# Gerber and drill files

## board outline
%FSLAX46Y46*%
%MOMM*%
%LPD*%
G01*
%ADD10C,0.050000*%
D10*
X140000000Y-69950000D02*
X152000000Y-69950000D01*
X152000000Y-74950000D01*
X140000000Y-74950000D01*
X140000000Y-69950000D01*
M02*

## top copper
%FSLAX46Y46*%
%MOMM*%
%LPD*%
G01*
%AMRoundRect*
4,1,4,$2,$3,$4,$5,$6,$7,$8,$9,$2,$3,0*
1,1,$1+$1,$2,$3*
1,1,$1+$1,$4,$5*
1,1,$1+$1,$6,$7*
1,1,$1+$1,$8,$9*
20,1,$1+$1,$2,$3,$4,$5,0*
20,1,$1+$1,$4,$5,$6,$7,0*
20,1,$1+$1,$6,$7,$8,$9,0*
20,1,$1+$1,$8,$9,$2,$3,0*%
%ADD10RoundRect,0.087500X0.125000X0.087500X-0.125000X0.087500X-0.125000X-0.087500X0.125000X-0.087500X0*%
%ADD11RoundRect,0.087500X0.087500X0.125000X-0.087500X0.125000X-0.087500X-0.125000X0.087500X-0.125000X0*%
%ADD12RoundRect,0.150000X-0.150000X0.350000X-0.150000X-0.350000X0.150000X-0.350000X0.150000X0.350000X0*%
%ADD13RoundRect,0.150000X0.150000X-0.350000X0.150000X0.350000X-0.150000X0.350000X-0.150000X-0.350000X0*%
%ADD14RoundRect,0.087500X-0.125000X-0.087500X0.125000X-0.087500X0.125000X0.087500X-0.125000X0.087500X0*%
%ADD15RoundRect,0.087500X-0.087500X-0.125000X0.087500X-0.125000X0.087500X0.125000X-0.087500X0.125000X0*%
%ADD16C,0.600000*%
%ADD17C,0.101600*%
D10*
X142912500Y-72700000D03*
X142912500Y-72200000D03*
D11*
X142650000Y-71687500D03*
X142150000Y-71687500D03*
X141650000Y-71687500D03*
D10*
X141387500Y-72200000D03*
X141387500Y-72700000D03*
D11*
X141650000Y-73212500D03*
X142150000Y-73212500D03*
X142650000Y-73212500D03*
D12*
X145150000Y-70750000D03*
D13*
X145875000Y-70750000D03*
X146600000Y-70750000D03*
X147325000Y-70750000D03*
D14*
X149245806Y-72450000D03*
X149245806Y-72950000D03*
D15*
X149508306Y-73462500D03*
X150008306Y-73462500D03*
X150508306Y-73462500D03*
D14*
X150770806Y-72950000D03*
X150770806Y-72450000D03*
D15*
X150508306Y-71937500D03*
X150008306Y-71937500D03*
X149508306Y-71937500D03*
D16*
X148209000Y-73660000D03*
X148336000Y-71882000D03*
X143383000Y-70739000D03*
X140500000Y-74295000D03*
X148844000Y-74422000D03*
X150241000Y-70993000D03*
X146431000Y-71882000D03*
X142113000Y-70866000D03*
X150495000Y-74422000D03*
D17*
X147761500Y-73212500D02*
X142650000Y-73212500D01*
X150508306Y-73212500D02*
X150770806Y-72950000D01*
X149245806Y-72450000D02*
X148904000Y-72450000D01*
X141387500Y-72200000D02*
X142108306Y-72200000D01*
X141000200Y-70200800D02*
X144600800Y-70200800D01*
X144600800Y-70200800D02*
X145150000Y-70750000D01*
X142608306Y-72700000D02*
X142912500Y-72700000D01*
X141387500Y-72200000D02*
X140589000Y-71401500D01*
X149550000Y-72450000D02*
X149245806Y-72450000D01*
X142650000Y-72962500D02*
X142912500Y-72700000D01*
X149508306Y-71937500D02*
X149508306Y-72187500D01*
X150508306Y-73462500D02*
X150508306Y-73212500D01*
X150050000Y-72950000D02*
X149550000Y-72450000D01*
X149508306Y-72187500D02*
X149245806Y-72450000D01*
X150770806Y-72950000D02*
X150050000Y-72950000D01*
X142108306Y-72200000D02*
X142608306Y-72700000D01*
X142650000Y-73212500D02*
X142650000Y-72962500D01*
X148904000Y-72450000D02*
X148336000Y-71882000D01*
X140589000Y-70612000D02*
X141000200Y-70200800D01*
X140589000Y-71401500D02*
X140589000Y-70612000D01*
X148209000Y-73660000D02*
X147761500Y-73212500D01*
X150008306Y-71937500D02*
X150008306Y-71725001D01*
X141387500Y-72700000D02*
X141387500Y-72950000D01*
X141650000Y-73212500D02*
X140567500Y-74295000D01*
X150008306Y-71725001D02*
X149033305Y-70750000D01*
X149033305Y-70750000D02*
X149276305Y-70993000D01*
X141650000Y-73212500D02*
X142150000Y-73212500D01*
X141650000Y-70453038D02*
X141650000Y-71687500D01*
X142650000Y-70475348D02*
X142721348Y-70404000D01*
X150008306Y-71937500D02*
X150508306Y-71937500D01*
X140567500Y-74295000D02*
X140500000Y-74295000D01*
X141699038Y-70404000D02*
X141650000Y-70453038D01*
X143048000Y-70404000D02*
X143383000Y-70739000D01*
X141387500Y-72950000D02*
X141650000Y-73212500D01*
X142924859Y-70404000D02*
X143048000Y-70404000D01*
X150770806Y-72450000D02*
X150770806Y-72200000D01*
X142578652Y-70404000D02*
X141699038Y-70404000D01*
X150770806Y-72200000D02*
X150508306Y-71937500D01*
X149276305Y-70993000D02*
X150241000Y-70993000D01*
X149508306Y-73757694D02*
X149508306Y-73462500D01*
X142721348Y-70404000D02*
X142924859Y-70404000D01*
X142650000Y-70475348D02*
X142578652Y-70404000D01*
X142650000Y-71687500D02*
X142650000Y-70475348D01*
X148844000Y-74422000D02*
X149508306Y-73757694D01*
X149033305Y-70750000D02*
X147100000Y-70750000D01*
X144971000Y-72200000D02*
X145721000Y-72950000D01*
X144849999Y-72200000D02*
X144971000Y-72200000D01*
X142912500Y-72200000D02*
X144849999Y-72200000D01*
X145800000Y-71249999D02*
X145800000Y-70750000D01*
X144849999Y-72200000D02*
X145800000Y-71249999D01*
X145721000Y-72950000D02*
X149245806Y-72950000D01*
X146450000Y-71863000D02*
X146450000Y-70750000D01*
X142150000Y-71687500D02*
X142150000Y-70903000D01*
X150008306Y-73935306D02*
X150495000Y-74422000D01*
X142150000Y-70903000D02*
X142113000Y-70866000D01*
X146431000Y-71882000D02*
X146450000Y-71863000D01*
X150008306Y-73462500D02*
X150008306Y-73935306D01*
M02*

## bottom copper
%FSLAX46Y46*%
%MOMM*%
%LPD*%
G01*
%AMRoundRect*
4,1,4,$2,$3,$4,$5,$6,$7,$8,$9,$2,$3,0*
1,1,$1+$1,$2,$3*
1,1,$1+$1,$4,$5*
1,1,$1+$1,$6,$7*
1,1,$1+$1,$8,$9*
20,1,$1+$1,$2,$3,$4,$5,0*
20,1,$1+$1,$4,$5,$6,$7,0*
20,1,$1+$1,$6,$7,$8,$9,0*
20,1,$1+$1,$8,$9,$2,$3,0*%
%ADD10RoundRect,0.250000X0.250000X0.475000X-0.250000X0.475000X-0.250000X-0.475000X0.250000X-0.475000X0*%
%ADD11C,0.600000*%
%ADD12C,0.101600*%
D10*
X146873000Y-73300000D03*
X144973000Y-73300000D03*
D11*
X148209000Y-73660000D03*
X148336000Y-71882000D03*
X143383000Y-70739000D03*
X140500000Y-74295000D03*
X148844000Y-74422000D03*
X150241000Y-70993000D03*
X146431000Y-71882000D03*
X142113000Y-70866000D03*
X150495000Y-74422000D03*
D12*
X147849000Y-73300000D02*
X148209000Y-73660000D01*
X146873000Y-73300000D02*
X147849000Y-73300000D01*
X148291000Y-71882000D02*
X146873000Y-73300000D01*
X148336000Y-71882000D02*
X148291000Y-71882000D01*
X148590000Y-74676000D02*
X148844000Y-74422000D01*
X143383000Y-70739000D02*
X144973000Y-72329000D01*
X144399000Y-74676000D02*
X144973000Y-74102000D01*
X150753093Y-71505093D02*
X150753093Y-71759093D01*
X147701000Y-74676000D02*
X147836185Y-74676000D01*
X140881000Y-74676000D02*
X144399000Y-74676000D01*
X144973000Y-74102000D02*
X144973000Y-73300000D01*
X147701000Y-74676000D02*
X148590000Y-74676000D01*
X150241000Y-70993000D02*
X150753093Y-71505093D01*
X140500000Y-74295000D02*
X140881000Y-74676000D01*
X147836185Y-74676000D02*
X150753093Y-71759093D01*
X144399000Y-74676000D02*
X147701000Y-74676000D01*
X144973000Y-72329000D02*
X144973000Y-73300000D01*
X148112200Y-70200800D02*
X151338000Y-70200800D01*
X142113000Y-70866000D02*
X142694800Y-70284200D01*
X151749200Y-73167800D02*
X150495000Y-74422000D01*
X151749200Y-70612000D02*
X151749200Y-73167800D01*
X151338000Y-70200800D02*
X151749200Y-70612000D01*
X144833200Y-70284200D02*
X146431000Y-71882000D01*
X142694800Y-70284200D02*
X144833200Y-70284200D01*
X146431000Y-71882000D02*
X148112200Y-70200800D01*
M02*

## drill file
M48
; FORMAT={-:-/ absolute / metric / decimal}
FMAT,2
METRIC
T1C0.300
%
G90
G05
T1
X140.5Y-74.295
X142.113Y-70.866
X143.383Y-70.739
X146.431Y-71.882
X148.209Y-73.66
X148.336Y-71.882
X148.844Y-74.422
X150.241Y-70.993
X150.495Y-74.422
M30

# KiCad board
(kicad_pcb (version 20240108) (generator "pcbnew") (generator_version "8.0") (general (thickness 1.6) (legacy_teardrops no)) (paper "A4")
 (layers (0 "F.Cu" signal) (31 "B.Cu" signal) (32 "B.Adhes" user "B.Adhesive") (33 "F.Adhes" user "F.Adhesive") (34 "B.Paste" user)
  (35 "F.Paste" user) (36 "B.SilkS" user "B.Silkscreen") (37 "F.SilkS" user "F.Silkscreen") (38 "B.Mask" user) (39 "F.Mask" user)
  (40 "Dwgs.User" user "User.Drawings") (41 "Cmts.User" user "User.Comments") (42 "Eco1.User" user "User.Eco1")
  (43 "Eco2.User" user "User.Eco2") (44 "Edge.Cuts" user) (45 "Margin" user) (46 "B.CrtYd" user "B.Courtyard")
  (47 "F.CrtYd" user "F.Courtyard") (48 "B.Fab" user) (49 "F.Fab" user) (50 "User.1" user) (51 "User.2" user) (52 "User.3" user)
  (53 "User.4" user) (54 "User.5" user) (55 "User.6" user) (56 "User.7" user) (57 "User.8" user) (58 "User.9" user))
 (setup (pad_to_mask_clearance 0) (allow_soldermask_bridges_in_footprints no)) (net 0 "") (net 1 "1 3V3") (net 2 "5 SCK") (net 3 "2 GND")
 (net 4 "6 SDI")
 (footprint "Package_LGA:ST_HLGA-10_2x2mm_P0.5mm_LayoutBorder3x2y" (layer "F.Cu") (at 142.15 72.45 180)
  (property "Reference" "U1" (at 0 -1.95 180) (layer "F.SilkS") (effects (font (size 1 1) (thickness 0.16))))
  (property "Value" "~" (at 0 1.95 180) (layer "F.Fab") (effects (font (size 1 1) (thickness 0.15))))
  (pad "1" smd roundrect (at -0.7625 -0.25 180) (size 0.425 0.35) (layers "F.Cu" "F.Paste" "F.Mask") (roundrect_rratio 0.25) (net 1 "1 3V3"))
  (pad "2" smd roundrect (at -0.7625 0.25 180) (size 0.425 0.35) (layers "F.Cu" "F.Paste" "F.Mask") (roundrect_rratio 0.25) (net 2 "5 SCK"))
  (pad "3" smd roundrect (at -0.5 0.7625 180) (size 0.35 0.425) (layers "F.Cu" "F.Paste" "F.Mask") (roundrect_rratio 0.25) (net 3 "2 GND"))
  (pad "4" smd roundrect (at 0 0.7625 180) (size 0.35 0.425) (layers "F.Cu" "F.Paste" "F.Mask") (roundrect_rratio 0.25) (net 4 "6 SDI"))
  (pad "5" smd roundrect (at 0.5 0.7625 180) (size 0.35 0.425) (layers "F.Cu" "F.Paste" "F.Mask") (roundrect_rratio 0.25) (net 3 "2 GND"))
  (pad "6" smd roundrect (at 0.7625 0.25 180) (size 0.425 0.35) (layers "F.Cu" "F.Paste" "F.Mask") (roundrect_rratio 0.25) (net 1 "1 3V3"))
  (pad "7" smd roundrect (at 0.7625 -0.25 180) (size 0.425 0.35) (layers "F.Cu" "F.Paste" "F.Mask") (roundrect_rratio 0.25) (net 3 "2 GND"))
  (pad "8" smd roundrect (at 0.5 -0.7625 180) (size 0.35 0.425) (layers "F.Cu" "F.Paste" "F.Mask") (roundrect_rratio 0.25) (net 3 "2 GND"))
  (pad "9" smd roundrect (at 0 -0.7625 180) (size 0.35 0.425) (layers "F.Cu" "F.Paste" "F.Mask") (roundrect_rratio 0.25) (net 3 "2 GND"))
  (pad "10" smd roundrect (at -0.5 -0.7625 180) (size 0.35 0.425) (layers "F.Cu" "F.Paste" "F.Mask") (roundrect_rratio 0.25) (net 1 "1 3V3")))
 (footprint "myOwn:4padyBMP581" (layer "F.Cu") (at 144.95 65)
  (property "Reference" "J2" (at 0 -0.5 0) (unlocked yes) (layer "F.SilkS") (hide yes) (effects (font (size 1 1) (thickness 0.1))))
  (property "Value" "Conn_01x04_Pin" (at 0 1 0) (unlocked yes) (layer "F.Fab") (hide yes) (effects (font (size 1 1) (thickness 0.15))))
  (pad "1" smd roundrect (at 0.2 5.75 270) (size 1 0.6) (layers "F.Cu" "F.Paste" "F.Mask") (roundrect_rratio 0.25) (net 1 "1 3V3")
   (thermal_bridge_angle 45))
  (pad "2" smd roundrect (at 0.925 5.75 90) (size 1 0.6) (layers "F.Cu" "F.Paste" "F.Mask") (roundrect_rratio 0.25) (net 2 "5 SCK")
   (thermal_bridge_angle 45))
  (pad "3" smd roundrect (at 1.65 5.75 90) (size 1 0.6) (layers "F.Cu" "F.Paste" "F.Mask") (roundrect_rratio 0.25) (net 4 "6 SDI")
   (thermal_bridge_angle 45))
  (pad "4" smd roundrect (at 2.375 5.75 90) (size 1 0.6) (layers "F.Cu" "F.Paste" "F.Mask") (roundrect_rratio 0.25) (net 3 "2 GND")
   (thermal_bridge_angle 45)))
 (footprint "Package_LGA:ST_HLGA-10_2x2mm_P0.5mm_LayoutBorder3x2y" (layer "F.Cu") (at 150.008306 72.7)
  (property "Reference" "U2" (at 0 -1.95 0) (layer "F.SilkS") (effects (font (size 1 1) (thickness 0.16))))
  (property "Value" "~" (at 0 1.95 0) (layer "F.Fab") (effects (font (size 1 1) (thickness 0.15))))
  (pad "1" smd roundrect (at -0.7625 -0.25) (size 0.425 0.35) (layers "F.Cu" "F.Paste" "F.Mask") (roundrect_rratio 0.25) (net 1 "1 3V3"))
  (pad "2" smd roundrect (at -0.7625 0.25) (size 0.425 0.35) (layers "F.Cu" "F.Paste" "F.Mask") (roundrect_rratio 0.25) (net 2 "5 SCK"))
  (pad "3" smd roundrect (at -0.5 0.7625) (size 0.35 0.425) (layers "F.Cu" "F.Paste" "F.Mask") (roundrect_rratio 0.25) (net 3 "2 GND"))
  (pad "4" smd roundrect (at 0 0.7625) (size 0.35 0.425) (layers "F.Cu" "F.Paste" "F.Mask") (roundrect_rratio 0.25) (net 4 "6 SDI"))
  (pad "5" smd roundrect (at 0.5 0.7625) (size 0.35 0.425) (layers "F.Cu" "F.Paste" "F.Mask") (roundrect_rratio 0.25) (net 1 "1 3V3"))
  (pad "6" smd roundrect (at 0.7625 0.25) (size 0.425 0.35) (layers "F.Cu" "F.Paste" "F.Mask") (roundrect_rratio 0.25) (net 1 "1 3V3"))
  (pad "7" smd roundrect (at 0.7625 -0.25) (size 0.425 0.35) (layers "F.Cu" "F.Paste" "F.Mask") (roundrect_rratio 0.25) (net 3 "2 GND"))
  (pad "8" smd roundrect (at 0.5 -0.7625) (size 0.35 0.425) (layers "F.Cu" "F.Paste" "F.Mask") (roundrect_rratio 0.25) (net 3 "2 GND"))
  (pad "9" smd roundrect (at 0 -0.7625) (size 0.35 0.425) (layers "F.Cu" "F.Paste" "F.Mask") (roundrect_rratio 0.25) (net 3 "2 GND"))
  (pad "10" smd roundrect (at -0.5 -0.7625) (size 0.35 0.425) (layers "F.Cu" "F.Paste" "F.Mask") (roundrect_rratio 0.25) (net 1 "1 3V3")))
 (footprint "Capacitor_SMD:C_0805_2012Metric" (layer "B.Cu") (at 145.923 73.3 180)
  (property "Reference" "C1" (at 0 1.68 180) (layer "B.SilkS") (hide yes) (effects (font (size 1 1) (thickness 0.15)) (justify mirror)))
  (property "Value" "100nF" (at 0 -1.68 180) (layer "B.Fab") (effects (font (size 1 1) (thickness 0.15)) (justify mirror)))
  (pad "1" smd roundrect (at -0.95 0 180) (size 1 1.45) (layers "B.Cu" "B.Paste" "B.Mask") (roundrect_rratio 0.25) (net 1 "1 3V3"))
  (pad "2" smd roundrect (at 0.95 0 180) (size 1 1.45) (layers "B.Cu" "B.Paste" "B.Mask") (roundrect_rratio 0.25) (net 3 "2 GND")))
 (gr_rect (start 140 69.95) (end 152 74.95) (stroke (width 0.05) (type default)) (fill none) (layer "Edge.Cuts"))
 (segment (start 147.7615 73.2125) (end 142.65 73.2125) (width 0.1016) (layer "F.Cu") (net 1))
 (segment (start 150.508306 73.2125) (end 150.770806 72.95) (width 0.1016) (layer "F.Cu") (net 1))
 (segment (start 149.245806 72.45) (end 148.904 72.45) (width 0.1016) (layer "F.Cu") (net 1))
 (segment (start 141.3875 72.2) (end 142.108306 72.2) (width 0.1016) (layer "F.Cu") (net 1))
 (segment (start 141.0002 70.2008) (end 144.6008 70.2008) (width 0.1016) (layer "F.Cu") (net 1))
 (segment (start 144.6008 70.2008) (end 145.15 70.75) (width 0.1016) (layer "F.Cu") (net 1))
 (segment (start 142.608306 72.7) (end 142.9125 72.7) (width 0.1016) (layer "F.Cu") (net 1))
 (segment (start 141.3875 72.2) (end 140.589 71.4015) (width 0.1016) (layer "F.Cu") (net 1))
 (segment (start 149.55 72.45) (end 149.245806 72.45) (width 0.1016) (layer "F.Cu") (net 1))
 (segment (start 142.65 72.9625) (end 142.9125 72.7) (width 0.1016) (layer "F.Cu") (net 1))
 (segment (start 149.508306 71.9375) (end 149.508306 72.1875) (width 0.1016) (layer "F.Cu") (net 1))
 (segment (start 150.508306 73.4625) (end 150.508306 73.2125) (width 0.1016) (layer "F.Cu") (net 1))
 (segment (start 150.05 72.95) (end 149.55 72.45) (width 0.1016) (layer "F.Cu") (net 1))
 (segment (start 149.508306 72.1875) (end 149.245806 72.45) (width 0.1016) (layer "F.Cu") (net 1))
 (segment (start 150.770806 72.95) (end 150.05 72.95) (width 0.1016) (layer "F.Cu") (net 1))
 (segment (start 142.108306 72.2) (end 142.608306 72.7) (width 0.1016) (layer "F.Cu") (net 1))
 (segment (start 142.65 73.2125) (end 142.65 72.9625) (width 0.1016) (layer "F.Cu") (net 1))
 (segment (start 148.904 72.45) (end 148.336 71.882) (width 0.1016) (layer "F.Cu") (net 1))
 (segment (start 140.589 70.612) (end 141.0002 70.2008) (width 0.1016) (layer "F.Cu") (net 1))
 (segment (start 140.589 71.4015) (end 140.589 70.612) (width 0.1016) (layer "F.Cu") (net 1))
 (segment (start 148.209 73.66) (end 147.7615 73.2125) (width 0.1016) (layer "F.Cu") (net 1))
 (via (at 148.209 73.66) (size 0.6) (drill 0.3) (layers "F.Cu" "B.Cu") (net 1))
 (via (at 148.336 71.882) (size 0.6) (drill 0.3) (layers "F.Cu" "B.Cu") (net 1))
 (segment (start 147.849 73.3) (end 148.209 73.66) (width 0.1016) (layer "B.Cu") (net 1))
 (segment (start 146.873 73.3) (end 147.849 73.3) (width 0.1016) (layer "B.Cu") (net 1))
 (segment (start 148.291 71.882) (end 146.873 73.3) (width 0.1016) (layer "B.Cu") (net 1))
 (segment (start 148.336 71.882) (end 148.291 71.882) (width 0.1016) (layer "B.Cu") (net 1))
 (segment (start 150.008306 71.9375) (end 150.008306 71.725001) (width 0.1016) (layer "F.Cu") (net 3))
 (segment (start 141.3875 72.7) (end 141.3875 72.95) (width 0.1016) (layer "F.Cu") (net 3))
 (segment (start 141.65 73.2125) (end 140.5675 74.295) (width 0.1016) (layer "F.Cu") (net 3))
 (segment (start 150.008306 71.725001) (end 149.033305 70.75) (width 0.1016) (layer "F.Cu") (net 3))
 (segment (start 149.033305 70.75) (end 149.276305 70.993) (width 0.1016) (layer "F.Cu") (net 3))
 (segment (start 141.65 73.2125) (end 142.15 73.2125) (width 0.1016) (layer "F.Cu") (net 3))
 (segment (start 141.65 70.453038) (end 141.65 71.6875) (width 0.1016) (layer "F.Cu") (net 3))
 (segment (start 142.65 70.475348) (end 142.721348 70.404) (width 0.1016) (layer "F.Cu") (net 3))
 (segment (start 150.008306 71.9375) (end 150.508306 71.9375) (width 0.1016) (layer "F.Cu") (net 3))
 (segment (start 140.5675 74.295) (end 140.5 74.295) (width 0.1016) (layer "F.Cu") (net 3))
 (segment (start 141.699038 70.404) (end 141.65 70.453038) (width 0.1016) (layer "F.Cu") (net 3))
 (segment (start 143.048 70.404) (end 143.383 70.739) (width 0.1016) (layer "F.Cu") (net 3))
 (segment (start 141.3875 72.95) (end 141.65 73.2125) (width 0.1016) (layer "F.Cu") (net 3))
 (segment (start 142.924859 70.404) (end 143.048 70.404) (width 0.1016) (layer "F.Cu") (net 3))
 (segment (start 150.770806 72.45) (end 150.770806 72.2) (width 0.1016) (layer "F.Cu") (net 3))
 (segment (start 142.578652 70.404) (end 141.699038 70.404) (width 0.1016) (layer "F.Cu") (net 3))
 (segment (start 150.770806 72.2) (end 150.508306 71.9375) (width 0.1016) (layer "F.Cu") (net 3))
 (segment (start 149.276305 70.993) (end 150.241 70.993) (width 0.1016) (layer "F.Cu") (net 3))
 (segment (start 149.508306 73.757694) (end 149.508306 73.4625) (width 0.1016) (layer "F.Cu") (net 3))
 (segment (start 142.721348 70.404) (end 142.924859 70.404) (width 0.1016) (layer "F.Cu") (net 3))
 (segment (start 142.65 70.475348) (end 142.578652 70.404) (width 0.1016) (layer "F.Cu") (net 3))
 (segment (start 142.65 71.6875) (end 142.65 70.475348) (width 0.1016) (layer "F.Cu") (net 3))
 (segment (start 148.844 74.422) (end 149.508306 73.757694) (width 0.1016) (layer "F.Cu") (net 3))
 (segment (start 149.033305 70.75) (end 147.1 70.75) (width 0.1016) (layer "F.Cu") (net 3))
 (via (at 143.383 70.739) (size 0.6) (drill 0.3) (layers "F.Cu" "B.Cu") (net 3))
 (via (at 140.5 74.295) (size 0.6) (drill 0.3) (layers "F.Cu" "B.Cu") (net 3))
 (via (at 148.844 74.422) (size 0.6) (drill 0.3) (layers "F.Cu" "B.Cu") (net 3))
 (via (at 150.241 70.993) (size 0.6) (drill 0.3) (layers "F.Cu" "B.Cu") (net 3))
 (segment (start 148.59 74.676) (end 148.844 74.422) (width 0.1016) (layer "B.Cu") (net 3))
 (segment (start 143.383 70.739) (end 144.973 72.329) (width 0.1016) (layer "B.Cu") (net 3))
 (segment (start 144.399 74.676) (end 144.973 74.102) (width 0.1016) (layer "B.Cu") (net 3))
 (segment (start 150.753093 71.505093) (end 150.753093 71.759093) (width 0.1016) (layer "B.Cu") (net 3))
 (segment (start 147.701 74.676) (end 147.836185 74.676) (width 0.1016) (layer "B.Cu") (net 3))
 (segment (start 140.881 74.676) (end 144.399 74.676) (width 0.1016) (layer "B.Cu") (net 3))
 (segment (start 144.973 74.102) (end 144.973 73.3) (width 0.1016) (layer "B.Cu") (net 3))
 (segment (start 147.701 74.676) (end 148.59 74.676) (width 0.1016) (layer "B.Cu") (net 3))
 (segment (start 150.241 70.993) (end 150.753093 71.505093) (width 0.1016) (layer "B.Cu") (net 3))
 (segment (start 140.5 74.295) (end 140.881 74.676) (width 0.1016) (layer "B.Cu") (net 3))
 (segment (start 147.836185 74.676) (end 150.753093 71.759093) (width 0.1016) (layer "B.Cu") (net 3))
 (segment (start 144.399 74.676) (end 147.701 74.676) (width 0.1016) (layer "B.Cu") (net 3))
 (segment (start 144.973 72.329) (end 144.973 73.3) (width 0.1016) (layer "B.Cu") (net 3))
 (segment (start 144.971 72.2) (end 145.721 72.95) (width 0.1016) (layer "F.Cu") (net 2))
 (segment (start 144.849999 72.2) (end 144.971 72.2) (width 0.1016) (layer "F.Cu") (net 2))
 (segment (start 142.9125 72.2) (end 144.849999 72.2) (width 0.1016) (layer "F.Cu") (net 2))
 (segment (start 145.8 71.249999) (end 145.8 70.75) (width 0.1016) (layer "F.Cu") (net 2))
 (segment (start 144.849999 72.2) (end 145.8 71.249999) (width 0.1016) (layer "F.Cu") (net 2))
 (segment (start 145.721 72.95) (end 149.245806 72.95) (width 0.1016) (layer "F.Cu") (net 2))
 (segment (start 146.45 71.863) (end 146.45 70.75) (width 0.1016) (layer "F.Cu") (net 4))
 (segment (start 142.15 71.6875) (end 142.15 70.903) (width 0.1016) (layer "F.Cu") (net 4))
 (segment (start 150.008306 73.935306) (end 150.495 74.422) (width 0.1016) (layer "F.Cu") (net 4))
 (segment (start 142.15 70.903) (end 142.113 70.866) (width 0.1016) (layer "F.Cu") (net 4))
 (segment (start 146.431 71.882) (end 146.45 71.863) (width 0.1016) (layer "F.Cu") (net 4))
 (segment (start 150.008306 73.4625) (end 150.008306 73.935306) (width 0.1016) (layer "F.Cu") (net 4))
 (via (at 146.431 71.882) (size 0.6) (drill 0.3) (layers "F.Cu" "B.Cu") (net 4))
 (via (at 142.113 70.866) (size 0.6) (drill 0.3) (layers "F.Cu" "B.Cu") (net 4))
 (via (at 150.495 74.422) (size 0.6) (drill 0.3) (layers "F.Cu" "B.Cu") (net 4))
 (segment (start 148.1122 70.2008) (end 151.338 70.2008) (width 0.1016) (layer "B.Cu") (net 4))
 (segment (start 142.113 70.866) (end 142.6948 70.2842) (width 0.1016) (layer "B.Cu") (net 4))
 (segment (start 151.7492 73.1678) (end 150.495 74.422) (width 0.1016) (layer "B.Cu") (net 4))
 (segment (start 151.7492 70.612) (end 151.7492 73.1678) (width 0.1016) (layer "B.Cu") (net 4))
 (segment (start 151.338 70.2008) (end 151.7492 70.612) (width 0.1016) (layer "B.Cu") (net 4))
 (segment (start 144.8332 70.2842) (end 146.431 71.882) (width 0.1016) (layer "B.Cu") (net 4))
 (segment (start 142.6948 70.2842) (end 144.8332 70.2842) (width 0.1016) (layer "B.Cu") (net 4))
 (segment (start 146.431 71.882) (end 148.1122 70.2008) (width 0.1016) (layer "B.Cu") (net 4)))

